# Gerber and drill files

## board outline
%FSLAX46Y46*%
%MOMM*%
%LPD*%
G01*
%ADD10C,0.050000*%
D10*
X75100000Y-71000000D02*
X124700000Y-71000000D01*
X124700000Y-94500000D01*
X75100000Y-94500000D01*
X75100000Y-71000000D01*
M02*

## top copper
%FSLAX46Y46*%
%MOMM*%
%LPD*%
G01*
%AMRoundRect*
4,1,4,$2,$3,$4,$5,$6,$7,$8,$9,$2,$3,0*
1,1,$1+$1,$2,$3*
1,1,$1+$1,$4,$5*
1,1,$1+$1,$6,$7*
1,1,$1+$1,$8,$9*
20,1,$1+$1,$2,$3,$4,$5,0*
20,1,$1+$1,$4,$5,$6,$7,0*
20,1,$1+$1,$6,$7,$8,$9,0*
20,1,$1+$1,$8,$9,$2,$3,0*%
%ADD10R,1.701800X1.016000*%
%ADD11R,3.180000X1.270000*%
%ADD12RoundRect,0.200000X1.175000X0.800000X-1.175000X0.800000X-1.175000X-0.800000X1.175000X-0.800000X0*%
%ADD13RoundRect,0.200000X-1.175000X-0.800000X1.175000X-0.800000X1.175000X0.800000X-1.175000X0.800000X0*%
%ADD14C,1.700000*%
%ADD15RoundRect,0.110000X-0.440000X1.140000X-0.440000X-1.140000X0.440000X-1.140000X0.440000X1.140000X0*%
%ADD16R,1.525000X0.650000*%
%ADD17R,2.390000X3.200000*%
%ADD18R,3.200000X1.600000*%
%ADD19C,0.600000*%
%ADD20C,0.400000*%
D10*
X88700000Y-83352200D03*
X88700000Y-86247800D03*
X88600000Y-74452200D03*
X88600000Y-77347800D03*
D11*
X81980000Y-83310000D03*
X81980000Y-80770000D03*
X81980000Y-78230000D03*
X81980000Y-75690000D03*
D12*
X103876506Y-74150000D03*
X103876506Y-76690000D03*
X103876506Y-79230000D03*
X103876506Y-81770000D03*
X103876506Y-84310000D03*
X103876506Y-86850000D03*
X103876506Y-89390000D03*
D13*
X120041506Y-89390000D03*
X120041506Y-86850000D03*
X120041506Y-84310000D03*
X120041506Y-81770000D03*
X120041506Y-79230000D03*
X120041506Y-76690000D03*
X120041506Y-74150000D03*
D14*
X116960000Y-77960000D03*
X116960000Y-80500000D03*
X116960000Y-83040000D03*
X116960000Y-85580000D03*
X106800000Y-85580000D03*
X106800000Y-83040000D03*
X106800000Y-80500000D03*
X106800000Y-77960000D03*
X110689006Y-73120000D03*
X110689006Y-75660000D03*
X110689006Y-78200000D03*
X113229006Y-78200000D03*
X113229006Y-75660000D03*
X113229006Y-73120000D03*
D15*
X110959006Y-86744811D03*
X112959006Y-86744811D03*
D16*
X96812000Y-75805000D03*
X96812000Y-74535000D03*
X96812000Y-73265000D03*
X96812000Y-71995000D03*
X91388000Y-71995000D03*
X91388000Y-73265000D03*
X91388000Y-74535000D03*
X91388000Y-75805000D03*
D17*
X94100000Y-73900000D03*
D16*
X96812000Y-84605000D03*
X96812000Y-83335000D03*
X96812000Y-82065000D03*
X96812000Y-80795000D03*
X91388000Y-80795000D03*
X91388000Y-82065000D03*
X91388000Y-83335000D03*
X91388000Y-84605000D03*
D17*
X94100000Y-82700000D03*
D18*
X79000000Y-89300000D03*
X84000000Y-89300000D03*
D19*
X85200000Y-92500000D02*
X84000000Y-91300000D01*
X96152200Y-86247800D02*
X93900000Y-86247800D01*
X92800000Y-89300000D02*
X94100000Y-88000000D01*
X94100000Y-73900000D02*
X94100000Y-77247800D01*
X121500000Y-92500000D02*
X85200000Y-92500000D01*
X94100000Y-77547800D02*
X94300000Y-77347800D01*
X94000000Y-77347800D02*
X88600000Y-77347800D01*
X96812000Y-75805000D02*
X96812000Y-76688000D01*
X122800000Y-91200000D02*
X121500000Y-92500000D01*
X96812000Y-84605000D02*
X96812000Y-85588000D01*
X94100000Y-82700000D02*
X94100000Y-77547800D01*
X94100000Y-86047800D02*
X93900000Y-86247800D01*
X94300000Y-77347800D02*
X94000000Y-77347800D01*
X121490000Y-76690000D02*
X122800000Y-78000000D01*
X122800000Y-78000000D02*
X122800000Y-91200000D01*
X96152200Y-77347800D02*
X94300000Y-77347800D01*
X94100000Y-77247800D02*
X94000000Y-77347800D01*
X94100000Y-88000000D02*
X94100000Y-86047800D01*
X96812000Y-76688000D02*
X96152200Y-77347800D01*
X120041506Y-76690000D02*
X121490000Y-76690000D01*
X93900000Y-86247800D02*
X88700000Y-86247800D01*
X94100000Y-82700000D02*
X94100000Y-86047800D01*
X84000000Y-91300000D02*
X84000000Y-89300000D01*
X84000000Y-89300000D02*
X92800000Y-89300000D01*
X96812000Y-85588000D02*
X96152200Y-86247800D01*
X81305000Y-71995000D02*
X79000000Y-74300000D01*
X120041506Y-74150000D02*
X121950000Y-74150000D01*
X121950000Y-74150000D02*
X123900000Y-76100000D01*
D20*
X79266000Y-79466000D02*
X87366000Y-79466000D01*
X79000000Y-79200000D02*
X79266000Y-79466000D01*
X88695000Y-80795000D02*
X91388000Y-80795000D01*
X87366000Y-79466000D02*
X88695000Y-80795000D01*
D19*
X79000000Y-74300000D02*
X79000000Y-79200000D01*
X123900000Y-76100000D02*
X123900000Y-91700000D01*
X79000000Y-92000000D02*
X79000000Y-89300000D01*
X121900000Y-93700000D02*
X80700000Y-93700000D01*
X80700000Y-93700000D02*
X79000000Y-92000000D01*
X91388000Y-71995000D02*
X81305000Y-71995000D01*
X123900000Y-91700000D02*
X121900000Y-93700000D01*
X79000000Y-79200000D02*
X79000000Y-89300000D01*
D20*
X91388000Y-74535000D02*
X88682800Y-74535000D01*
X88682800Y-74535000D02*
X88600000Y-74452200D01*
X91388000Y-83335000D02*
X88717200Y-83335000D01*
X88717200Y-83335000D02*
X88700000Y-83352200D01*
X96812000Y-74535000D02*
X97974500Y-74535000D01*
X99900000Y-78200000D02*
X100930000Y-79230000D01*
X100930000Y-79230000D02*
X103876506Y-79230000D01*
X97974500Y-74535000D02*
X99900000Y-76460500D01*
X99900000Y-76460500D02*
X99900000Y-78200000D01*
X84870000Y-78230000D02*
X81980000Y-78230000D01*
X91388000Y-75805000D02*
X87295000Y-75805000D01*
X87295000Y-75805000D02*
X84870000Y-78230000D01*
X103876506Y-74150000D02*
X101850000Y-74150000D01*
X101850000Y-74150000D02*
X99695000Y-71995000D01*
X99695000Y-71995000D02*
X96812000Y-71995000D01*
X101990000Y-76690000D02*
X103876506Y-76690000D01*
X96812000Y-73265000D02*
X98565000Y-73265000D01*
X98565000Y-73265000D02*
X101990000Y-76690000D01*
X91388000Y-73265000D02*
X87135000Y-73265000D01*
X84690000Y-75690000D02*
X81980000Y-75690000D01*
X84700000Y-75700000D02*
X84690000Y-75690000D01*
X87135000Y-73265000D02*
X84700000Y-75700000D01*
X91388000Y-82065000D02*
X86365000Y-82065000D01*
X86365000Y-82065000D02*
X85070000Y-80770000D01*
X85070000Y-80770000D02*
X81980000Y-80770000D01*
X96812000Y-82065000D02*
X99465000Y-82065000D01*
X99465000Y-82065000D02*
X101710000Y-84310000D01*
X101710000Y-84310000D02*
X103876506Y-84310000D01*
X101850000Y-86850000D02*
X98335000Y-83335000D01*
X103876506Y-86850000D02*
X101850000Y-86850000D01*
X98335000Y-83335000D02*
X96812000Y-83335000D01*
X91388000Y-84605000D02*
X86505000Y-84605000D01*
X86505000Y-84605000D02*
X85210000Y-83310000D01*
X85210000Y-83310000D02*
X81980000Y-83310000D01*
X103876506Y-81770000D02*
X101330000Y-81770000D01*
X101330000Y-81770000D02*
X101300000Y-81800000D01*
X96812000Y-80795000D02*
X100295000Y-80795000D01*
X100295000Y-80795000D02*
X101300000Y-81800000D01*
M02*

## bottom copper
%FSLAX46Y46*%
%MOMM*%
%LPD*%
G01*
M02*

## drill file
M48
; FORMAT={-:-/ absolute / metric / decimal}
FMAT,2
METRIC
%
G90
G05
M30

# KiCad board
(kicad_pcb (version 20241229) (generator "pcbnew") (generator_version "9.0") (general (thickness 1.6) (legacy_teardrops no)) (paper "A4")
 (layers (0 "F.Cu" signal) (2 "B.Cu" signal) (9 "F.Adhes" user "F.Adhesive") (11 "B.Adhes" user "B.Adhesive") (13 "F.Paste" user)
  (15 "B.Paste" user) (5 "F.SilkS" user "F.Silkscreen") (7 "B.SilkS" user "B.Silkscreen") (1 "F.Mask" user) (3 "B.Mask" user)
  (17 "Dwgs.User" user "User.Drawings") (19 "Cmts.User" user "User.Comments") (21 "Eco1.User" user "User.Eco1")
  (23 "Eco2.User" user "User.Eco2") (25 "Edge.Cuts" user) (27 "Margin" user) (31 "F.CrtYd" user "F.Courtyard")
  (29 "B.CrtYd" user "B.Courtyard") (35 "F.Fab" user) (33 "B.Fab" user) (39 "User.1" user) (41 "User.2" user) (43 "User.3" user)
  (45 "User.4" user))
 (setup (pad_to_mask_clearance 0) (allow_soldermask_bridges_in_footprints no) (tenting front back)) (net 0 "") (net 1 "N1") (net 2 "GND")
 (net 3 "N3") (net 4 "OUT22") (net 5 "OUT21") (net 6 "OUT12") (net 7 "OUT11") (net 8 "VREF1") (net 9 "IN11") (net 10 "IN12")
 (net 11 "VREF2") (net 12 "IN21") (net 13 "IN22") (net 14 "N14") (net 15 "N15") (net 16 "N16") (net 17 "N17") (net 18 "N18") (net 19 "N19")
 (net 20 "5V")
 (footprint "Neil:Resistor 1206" (layer "F.Cu") (at 88.7 84.8 -90)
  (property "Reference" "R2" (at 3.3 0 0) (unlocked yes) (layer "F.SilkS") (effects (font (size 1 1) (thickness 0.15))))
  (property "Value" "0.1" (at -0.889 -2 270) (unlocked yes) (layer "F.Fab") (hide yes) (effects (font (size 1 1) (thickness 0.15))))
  (pad "1" smd rect (at -1.4478 0 270) (size 1.016 1.7018) (layers "F.Cu" "F.Mask" "F.Paste") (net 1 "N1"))
  (pad "2" smd rect (at 1.4478 0 270) (size 1.016 1.7018) (layers "F.Cu" "F.Mask" "F.Paste") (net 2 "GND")))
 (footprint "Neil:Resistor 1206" (layer "F.Cu") (at 88.6 75.9 -90)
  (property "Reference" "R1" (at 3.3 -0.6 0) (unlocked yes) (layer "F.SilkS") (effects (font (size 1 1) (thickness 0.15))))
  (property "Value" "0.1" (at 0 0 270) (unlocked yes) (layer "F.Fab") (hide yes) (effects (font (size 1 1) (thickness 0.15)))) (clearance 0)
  (pad "1" smd rect (at -1.4478 0 270) (size 1.016 1.7018) (layers "F.Cu" "F.Mask" "F.Paste") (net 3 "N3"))
  (pad "2" smd rect (at 1.4478 0 270) (size 1.016 1.7018) (layers "F.Cu" "F.Mask" "F.Paste") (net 2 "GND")))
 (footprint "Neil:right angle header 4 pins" (layer "F.Cu") (at 76.7 79.5 90)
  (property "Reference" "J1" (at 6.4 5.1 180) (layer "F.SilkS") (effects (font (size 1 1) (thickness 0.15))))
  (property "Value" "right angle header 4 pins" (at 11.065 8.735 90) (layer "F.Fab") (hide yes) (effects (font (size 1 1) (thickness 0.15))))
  (pad "01" smd rect (at -3.81 5.28 90) (size 1.27 3.18) (layers "F.Cu" "F.Mask" "F.Paste") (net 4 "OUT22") (solder_mask_margin 0.102))
  (pad "02" smd rect (at -1.27 5.28 90) (size 1.27 3.18) (layers "F.Cu" "F.Mask" "F.Paste") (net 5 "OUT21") (solder_mask_margin 0.102))
  (pad "03" smd rect (at 1.27 5.28 90) (size 1.27 3.18) (layers "F.Cu" "F.Mask" "F.Paste") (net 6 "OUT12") (solder_mask_margin 0.102))
  (pad "04" smd rect (at 3.81 5.28 90) (size 1.27 3.18) (layers "F.Cu" "F.Mask" "F.Paste") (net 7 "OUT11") (solder_mask_margin 0.102)))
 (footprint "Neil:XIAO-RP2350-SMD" (layer "F.Cu") (at 111.876506 81.77)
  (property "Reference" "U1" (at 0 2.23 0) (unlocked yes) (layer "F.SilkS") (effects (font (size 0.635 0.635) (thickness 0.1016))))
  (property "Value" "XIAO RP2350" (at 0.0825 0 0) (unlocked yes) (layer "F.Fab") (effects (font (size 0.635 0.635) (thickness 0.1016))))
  (pad "1" smd roundrect (at -8 -7.62 180) (size 2.75 2) (layers "F.Cu" "F.Mask" "F.Paste") (roundrect_rratio 0.1) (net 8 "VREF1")
   (thermal_bridge_angle 45))
  (pad "2" smd roundrect (at -8 -5.08 180) (size 2.75 2) (layers "F.Cu" "F.Mask" "F.Paste") (roundrect_rratio 0.1) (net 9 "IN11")
   (thermal_bridge_angle 45))
  (pad "3" smd roundrect (at -8 -2.54 180) (size 2.75 2) (layers "F.Cu" "F.Mask" "F.Paste") (roundrect_rratio 0.1) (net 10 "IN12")
   (thermal_bridge_angle 45))
  (pad "4" smd roundrect (at -8 0 180) (size 2.75 2) (layers "F.Cu" "F.Mask" "F.Paste") (roundrect_rratio 0.1) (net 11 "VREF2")
   (thermal_bridge_angle 45))
  (pad "5" smd roundrect (at -8 2.54 180) (size 2.75 2) (layers "F.Cu" "F.Mask" "F.Paste") (roundrect_rratio 0.1) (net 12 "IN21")
   (thermal_bridge_angle 45))
  (pad "6" smd roundrect (at -8 5.08 180) (size 2.75 2) (layers "F.Cu" "F.Mask" "F.Paste") (roundrect_rratio 0.1) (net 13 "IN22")
   (thermal_bridge_angle 45))
  (pad "7" smd roundrect (at -8 7.62 180) (size 2.75 2) (layers "F.Cu" "F.Mask" "F.Paste") (roundrect_rratio 0.1) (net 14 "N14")
   (thermal_bridge_angle 45))
  (pad "8" smd roundrect (at 8.165 7.62) (size 2.75 2) (layers "F.Cu" "F.Mask" "F.Paste") (roundrect_rratio 0.1) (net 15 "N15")
   (thermal_bridge_angle 45))
  (pad "9" smd roundrect (at 8.165 5.08) (size 2.75 2) (layers "F.Cu" "F.Mask" "F.Paste") (roundrect_rratio 0.1) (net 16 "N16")
   (thermal_bridge_angle 45))
  (pad "10" smd roundrect (at 8.165 2.54) (size 2.75 2) (layers "F.Cu" "F.Mask" "F.Paste") (roundrect_rratio 0.1) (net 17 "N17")
   (thermal_bridge_angle 45))
  (pad "11" smd roundrect (at 8.165 0) (size 2.75 2) (layers "F.Cu" "F.Mask" "F.Paste") (roundrect_rratio 0.1) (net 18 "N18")
   (thermal_bridge_angle 45))
  (pad "12" smd roundrect (at 8.165 -2.54) (size 2.75 2) (layers "F.Cu" "F.Mask" "F.Paste") (roundrect_rratio 0.1) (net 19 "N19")
   (thermal_bridge_angle 45))
  (pad "13" smd roundrect (at 8.165 -5.08) (size 2.75 2) (layers "F.Cu" "F.Mask" "F.Paste") (roundrect_rratio 0.1) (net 2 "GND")
   (thermal_bridge_angle 45))
  (pad "14" smd roundrect (at 8.165 -7.62) (size 2.75 2) (layers "F.Cu" "F.Mask" "F.Paste") (roundrect_rratio 0.1) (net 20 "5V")
   (thermal_bridge_angle 45))
  (pad "15" smd circle (at 5.083494 -3.81 180) (size 1.7 1.7) (layers "F.Cu" "F.Mask" "F.Paste"))
  (pad "16" smd circle (at 5.083494 -1.27 180) (size 1.7 1.7) (layers "F.Cu" "F.Mask" "F.Paste"))
  (pad "17" smd circle (at 5.083494 1.27 180) (size 1.7 1.7) (layers "F.Cu" "F.Mask" "F.Paste"))
  (pad "18" smd circle (at 5.083494 3.81 180) (size 1.7 1.7) (layers "F.Cu" "F.Mask" "F.Paste"))
  (pad "19" smd circle (at -5.076506 3.81 180) (size 1.7 1.7) (layers "F.Cu" "F.Mask" "F.Paste"))
  (pad "20" smd circle (at -5.076506 1.27 180) (size 1.7 1.7) (layers "F.Cu" "F.Mask" "F.Paste"))
  (pad "21" smd circle (at -5.076506 -1.27 180) (size 1.7 1.7) (layers "F.Cu" "F.Mask" "F.Paste"))
  (pad "22" smd circle (at -5.076506 -3.81 180) (size 1.7 1.7) (layers "F.Cu" "F.Mask" "F.Paste"))
  (pad "23" smd circle (at -1.1875 -8.65 180) (size 1.7 1.7) (layers "F.Cu" "F.Mask" "F.Paste"))
  (pad "24" smd circle (at -1.1875 -6.11 180) (size 1.7 1.7) (layers "F.Cu" "F.Mask" "F.Paste"))
  (pad "25" smd circle (at -1.1875 -3.57 180) (size 1.7 1.7) (layers "F.Cu" "F.Mask" "F.Paste"))
  (pad "26" smd circle (at 1.3525 -3.57 180) (size 1.7 1.7) (layers "F.Cu" "F.Mask" "F.Paste"))
  (pad "27" smd circle (at 1.3525 -6.11 180) (size 1.7 1.7) (layers "F.Cu" "F.Mask" "F.Paste"))
  (pad "28" smd circle (at 1.3525 -8.65 180) (size 1.7 1.7) (layers "F.Cu" "F.Mask" "F.Paste"))
  (pad "29" smd roundrect (at -0.9175 4.974811 270) (size 2.5 1.1) (layers "F.Cu" "F.Mask" "F.Paste") (roundrect_rratio 0.1)
   (thermal_bridge_angle 45))
  (pad "30" smd roundrect (at 1.0825 4.974811 270) (size 2.5 1.1) (layers "F.Cu" "F.Mask" "F.Paste") (roundrect_rratio 0.1)
   (thermal_bridge_angle 45)))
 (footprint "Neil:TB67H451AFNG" (layer "F.Cu") (at 94.1 73.9 180)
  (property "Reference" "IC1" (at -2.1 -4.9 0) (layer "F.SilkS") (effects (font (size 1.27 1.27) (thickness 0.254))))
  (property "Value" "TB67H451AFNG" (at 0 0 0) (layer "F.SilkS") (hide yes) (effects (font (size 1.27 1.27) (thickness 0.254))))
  (pad "1" smd rect (at -2.712 -1.905 270) (size 0.65 1.525) (layers "F.Cu" "F.Mask" "F.Paste") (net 2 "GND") (thermal_bridge_angle 45))
  (pad "2" smd rect (at -2.712 -0.635 270) (size 0.65 1.525) (layers "F.Cu" "F.Mask" "F.Paste") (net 10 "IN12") (thermal_bridge_angle 45))
  (pad "3" smd rect (at -2.712 0.635 270) (size 0.65 1.525) (layers "F.Cu" "F.Mask" "F.Paste") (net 9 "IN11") (thermal_bridge_angle 45))
  (pad "4" smd rect (at -2.712 1.905 270) (size 0.65 1.525) (layers "F.Cu" "F.Mask" "F.Paste") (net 8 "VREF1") (thermal_bridge_angle 45))
  (pad "5" smd rect (at 2.712 1.905 270) (size 0.65 1.525) (layers "F.Cu" "F.Mask" "F.Paste") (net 20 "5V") (thermal_bridge_angle 45))
  (pad "6" smd rect (at 2.712 0.635 270) (size 0.65 1.525) (layers "F.Cu" "F.Mask" "F.Paste") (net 7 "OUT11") (thermal_bridge_angle 45))
  (pad "7" smd rect (at 2.712 -0.635 270) (size 0.65 1.525) (layers "F.Cu" "F.Mask" "F.Paste") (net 3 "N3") (thermal_bridge_angle 45))
  (pad "8" smd rect (at 2.712 -1.905 270) (size 0.65 1.525) (layers "F.Cu" "F.Mask" "F.Paste") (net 6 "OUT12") (thermal_bridge_angle 45))
  (pad "9" smd rect (at 0 0 180) (size 2.39 3.2) (layers "F.Cu" "F.Mask" "F.Paste") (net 2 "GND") (thermal_bridge_angle 45)))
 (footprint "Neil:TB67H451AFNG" (layer "F.Cu") (at 94.1 82.7 180)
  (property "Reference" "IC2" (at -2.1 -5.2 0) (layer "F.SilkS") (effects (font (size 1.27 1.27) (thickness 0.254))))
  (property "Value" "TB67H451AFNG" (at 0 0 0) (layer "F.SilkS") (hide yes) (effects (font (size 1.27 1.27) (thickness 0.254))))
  (pad "1" smd rect (at -2.712 -1.905 270) (size 0.65 1.525) (layers "F.Cu" "F.Mask" "F.Paste") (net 2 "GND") (thermal_bridge_angle 45))
  (pad "2" smd rect (at -2.712 -0.635 270) (size 0.65 1.525) (layers "F.Cu" "F.Mask" "F.Paste") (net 13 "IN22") (thermal_bridge_angle 45))
  (pad "3" smd rect (at -2.712 0.635 270) (size 0.65 1.525) (layers "F.Cu" "F.Mask" "F.Paste") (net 12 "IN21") (thermal_bridge_angle 45))
  (pad "4" smd rect (at -2.712 1.905 270) (size 0.65 1.525) (layers "F.Cu" "F.Mask" "F.Paste") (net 11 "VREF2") (thermal_bridge_angle 45))
  (pad "5" smd rect (at 2.712 1.905 270) (size 0.65 1.525) (layers "F.Cu" "F.Mask" "F.Paste") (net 20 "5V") (thermal_bridge_angle 45))
  (pad "6" smd rect (at 2.712 0.635 270) (size 0.65 1.525) (layers "F.Cu" "F.Mask" "F.Paste") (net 5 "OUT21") (thermal_bridge_angle 45))
  (pad "7" smd rect (at 2.712 -0.635 270) (size 0.65 1.525) (layers "F.Cu" "F.Mask" "F.Paste") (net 1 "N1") (thermal_bridge_angle 45))
  (pad "8" smd rect (at 2.712 -1.905 270) (size 0.65 1.525) (layers "F.Cu" "F.Mask" "F.Paste") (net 4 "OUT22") (thermal_bridge_angle 45))
  (pad "9" smd rect (at 0 0 180) (size 2.39 3.2) (layers "F.Cu" "F.Mask" "F.Paste") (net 2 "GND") (thermal_bridge_angle 45)))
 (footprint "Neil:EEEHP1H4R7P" (layer "F.Cu") (at 81.5 89.3 -90)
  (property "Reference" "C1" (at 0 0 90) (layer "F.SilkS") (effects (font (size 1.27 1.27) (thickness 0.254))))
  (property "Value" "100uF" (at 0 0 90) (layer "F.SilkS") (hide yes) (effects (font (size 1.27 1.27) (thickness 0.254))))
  (pad "1" smd rect (at 0 2.5 270) (size 1.6 3.2) (layers "F.Cu" "F.Mask" "F.Paste") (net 20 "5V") (thermal_bridge_angle 45))
  (pad "2" smd rect (at 0 -2.5 270) (size 1.6 3.2) (layers "F.Cu" "F.Mask" "F.Paste") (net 2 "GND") (thermal_bridge_angle 45)))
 (gr_rect (start 75.1 71) (end 124.7 94.5) (stroke (width 0.05) (type default)) (fill no) (layer "Edge.Cuts"))
 (segment (start 85.2 92.5) (end 84 91.3) (width 0.6) (layer "F.Cu") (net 2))
 (segment (start 96.1522 86.2478) (end 93.9 86.2478) (width 0.6) (layer "F.Cu") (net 2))
 (segment (start 92.8 89.3) (end 94.1 88) (width 0.6) (layer "F.Cu") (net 2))
 (segment (start 94.1 73.9) (end 94.1 77.2478) (width 0.6) (layer "F.Cu") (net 2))
 (segment (start 121.5 92.5) (end 85.2 92.5) (width 0.6) (layer "F.Cu") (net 2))
 (segment (start 94.1 77.5478) (end 94.3 77.3478) (width 0.6) (layer "F.Cu") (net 2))
 (segment (start 94 77.3478) (end 88.6 77.3478) (width 0.6) (layer "F.Cu") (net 2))
 (segment (start 96.812 75.805) (end 96.812 76.688) (width 0.6) (layer "F.Cu") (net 2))
 (segment (start 122.8 91.2) (end 121.5 92.5) (width 0.6) (layer "F.Cu") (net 2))
 (segment (start 96.812 84.605) (end 96.812 85.588) (width 0.6) (layer "F.Cu") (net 2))
 (segment (start 94.1 82.7) (end 94.1 77.5478) (width 0.6) (layer "F.Cu") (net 2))
 (segment (start 94.1 86.0478) (end 93.9 86.2478) (width 0.6) (layer "F.Cu") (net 2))
 (segment (start 94.3 77.3478) (end 94 77.3478) (width 0.6) (layer "F.Cu") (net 2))
 (segment (start 121.49 76.69) (end 122.8 78) (width 0.6) (layer "F.Cu") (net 2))
 (segment (start 122.8 78) (end 122.8 91.2) (width 0.6) (layer "F.Cu") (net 2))
 (segment (start 96.1522 77.3478) (end 94.3 77.3478) (width 0.6) (layer "F.Cu") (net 2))
 (segment (start 94.1 77.2478) (end 94 77.3478) (width 0.6) (layer "F.Cu") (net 2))
 (segment (start 94.1 88) (end 94.1 86.0478) (width 0.6) (layer "F.Cu") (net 2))
 (segment (start 96.812 76.688) (end 96.1522 77.3478) (width 0.6) (layer "F.Cu") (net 2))
 (segment (start 120.041506 76.69) (end 121.49 76.69) (width 0.6) (layer "F.Cu") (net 2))
 (segment (start 93.9 86.2478) (end 88.7 86.2478) (width 0.6) (layer "F.Cu") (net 2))
 (segment (start 94.1 82.7) (end 94.1 86.0478) (width 0.6) (layer "F.Cu") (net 2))
 (segment (start 84 91.3) (end 84 89.3) (width 0.6) (layer "F.Cu") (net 2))
 (segment (start 84 89.3) (end 92.8 89.3) (width 0.6) (layer "F.Cu") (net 2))
 (segment (start 96.812 85.588) (end 96.1522 86.2478) (width 0.6) (layer "F.Cu") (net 2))
 (segment (start 81.305 71.995) (end 79 74.3) (width 0.6) (layer "F.Cu") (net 20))
 (segment (start 120.041506 74.15) (end 121.95 74.15) (width 0.6) (layer "F.Cu") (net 20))
 (segment (start 121.95 74.15) (end 123.9 76.1) (width 0.6) (layer "F.Cu") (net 20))
 (segment (start 79.266 79.466) (end 87.366 79.466) (width 0.4) (layer "F.Cu") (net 20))
 (segment (start 79 79.2) (end 79.266 79.466) (width 0.4) (layer "F.Cu") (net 20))
 (segment (start 88.695 80.795) (end 91.388 80.795) (width 0.4) (layer "F.Cu") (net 20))
 (segment (start 87.366 79.466) (end 88.695 80.795) (width 0.4) (layer "F.Cu") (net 20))
 (segment (start 79 74.3) (end 79 79.2) (width 0.6) (layer "F.Cu") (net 20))
 (segment (start 123.9 76.1) (end 123.9 91.7) (width 0.6) (layer "F.Cu") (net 20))
 (segment (start 79 92) (end 79 89.3) (width 0.6) (layer "F.Cu") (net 20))
 (segment (start 121.9 93.7) (end 80.7 93.7) (width 0.6) (layer "F.Cu") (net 20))
 (segment (start 80.7 93.7) (end 79 92) (width 0.6) (layer "F.Cu") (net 20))
 (segment (start 91.388 71.995) (end 81.305 71.995) (width 0.6) (layer "F.Cu") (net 20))
 (segment (start 123.9 91.7) (end 121.9 93.7) (width 0.6) (layer "F.Cu") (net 20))
 (segment (start 79 79.2) (end 79 89.3) (width 0.6) (layer "F.Cu") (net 20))
 (segment (start 91.388 74.535) (end 88.6828 74.535) (width 0.4) (layer "F.Cu") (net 3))
 (segment (start 88.6828 74.535) (end 88.6 74.4522) (width 0.4) (layer "F.Cu") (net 3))
 (segment (start 91.388 83.335) (end 88.7172 83.335) (width 0.4) (layer "F.Cu") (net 1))
 (segment (start 88.7172 83.335) (end 88.7 83.3522) (width 0.4) (layer "F.Cu") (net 1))
 (segment (start 96.812 74.535) (end 97.9745 74.535) (width 0.4) (layer "F.Cu") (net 10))
 (segment (start 99.9 78.2) (end 100.93 79.23) (width 0.4) (layer "F.Cu") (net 10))
 (segment (start 100.93 79.23) (end 103.876506 79.23) (width 0.4) (layer "F.Cu") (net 10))
 (segment (start 97.9745 74.535) (end 99.9 76.4605) (width 0.4) (layer "F.Cu") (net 10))
 (segment (start 99.9 76.4605) (end 99.9 78.2) (width 0.4) (layer "F.Cu") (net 10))
 (segment (start 84.87 78.23) (end 81.98 78.23) (width 0.4) (layer "F.Cu") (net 6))
 (segment (start 91.388 75.805) (end 87.295 75.805) (width 0.4) (layer "F.Cu") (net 6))
 (segment (start 87.295 75.805) (end 84.87 78.23) (width 0.4) (layer "F.Cu") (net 6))
 (segment (start 103.876506 74.15) (end 101.85 74.15) (width 0.4) (layer "F.Cu") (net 8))
 (segment (start 101.85 74.15) (end 99.695 71.995) (width 0.4) (layer "F.Cu") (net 8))
 (segment (start 99.695 71.995) (end 96.812 71.995) (width 0.4) (layer "F.Cu") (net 8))
 (segment (start 101.99 76.69) (end 103.876506 76.69) (width 0.4) (layer "F.Cu") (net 9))
 (segment (start 96.812 73.265) (end 98.565 73.265) (width 0.4) (layer "F.Cu") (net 9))
 (segment (start 98.565 73.265) (end 101.99 76.69) (width 0.4) (layer "F.Cu") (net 9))
 (segment (start 91.388 73.265) (end 87.135 73.265) (width 0.4) (layer "F.Cu") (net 7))
 (segment (start 84.69 75.69) (end 81.98 75.69) (width 0.4) (layer "F.Cu") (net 7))
 (segment (start 84.7 75.7) (end 84.69 75.69) (width 0.4) (layer "F.Cu") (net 7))
 (segment (start 87.135 73.265) (end 84.7 75.7) (width 0.4) (layer "F.Cu") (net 7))
 (segment (start 91.388 82.065) (end 86.365 82.065) (width 0.4) (layer "F.Cu") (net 5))
 (segment (start 86.365 82.065) (end 85.07 80.77) (width 0.4) (layer "F.Cu") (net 5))
 (segment (start 85.07 80.77) (end 81.98 80.77) (width 0.4) (layer "F.Cu") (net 5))
 (segment (start 96.812 82.065) (end 99.465 82.065) (width 0.4) (layer "F.Cu") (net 12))
 (segment (start 99.465 82.065) (end 101.71 84.31) (width 0.4) (layer "F.Cu") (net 12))
 (segment (start 101.71 84.31) (end 103.876506 84.31) (width 0.4) (layer "F.Cu") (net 12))
 (segment (start 101.85 86.85) (end 98.335 83.335) (width 0.4) (layer "F.Cu") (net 13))
 (segment (start 103.876506 86.85) (end 101.85 86.85) (width 0.4) (layer "F.Cu") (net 13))
 (segment (start 98.335 83.335) (end 96.812 83.335) (width 0.4) (layer "F.Cu") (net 13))
 (segment (start 91.388 84.605) (end 86.505 84.605) (width 0.4) (layer "F.Cu") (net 4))
 (segment (start 86.505 84.605) (end 85.21 83.31) (width 0.4) (layer "F.Cu") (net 4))
 (segment (start 85.21 83.31) (end 81.98 83.31) (width 0.4) (layer "F.Cu") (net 4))
 (segment (start 103.876506 81.77) (end 101.33 81.77) (width 0.4) (layer "F.Cu") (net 11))
 (segment (start 101.33 81.77) (end 101.3 81.8) (width 0.4) (layer "F.Cu") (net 11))
 (segment (start 96.812 80.795) (end 100.295 80.795) (width 0.4) (layer "F.Cu") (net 11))
 (segment (start 100.295 80.795) (end 101.3 81.8) (width 0.4) (layer "F.Cu") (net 11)))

